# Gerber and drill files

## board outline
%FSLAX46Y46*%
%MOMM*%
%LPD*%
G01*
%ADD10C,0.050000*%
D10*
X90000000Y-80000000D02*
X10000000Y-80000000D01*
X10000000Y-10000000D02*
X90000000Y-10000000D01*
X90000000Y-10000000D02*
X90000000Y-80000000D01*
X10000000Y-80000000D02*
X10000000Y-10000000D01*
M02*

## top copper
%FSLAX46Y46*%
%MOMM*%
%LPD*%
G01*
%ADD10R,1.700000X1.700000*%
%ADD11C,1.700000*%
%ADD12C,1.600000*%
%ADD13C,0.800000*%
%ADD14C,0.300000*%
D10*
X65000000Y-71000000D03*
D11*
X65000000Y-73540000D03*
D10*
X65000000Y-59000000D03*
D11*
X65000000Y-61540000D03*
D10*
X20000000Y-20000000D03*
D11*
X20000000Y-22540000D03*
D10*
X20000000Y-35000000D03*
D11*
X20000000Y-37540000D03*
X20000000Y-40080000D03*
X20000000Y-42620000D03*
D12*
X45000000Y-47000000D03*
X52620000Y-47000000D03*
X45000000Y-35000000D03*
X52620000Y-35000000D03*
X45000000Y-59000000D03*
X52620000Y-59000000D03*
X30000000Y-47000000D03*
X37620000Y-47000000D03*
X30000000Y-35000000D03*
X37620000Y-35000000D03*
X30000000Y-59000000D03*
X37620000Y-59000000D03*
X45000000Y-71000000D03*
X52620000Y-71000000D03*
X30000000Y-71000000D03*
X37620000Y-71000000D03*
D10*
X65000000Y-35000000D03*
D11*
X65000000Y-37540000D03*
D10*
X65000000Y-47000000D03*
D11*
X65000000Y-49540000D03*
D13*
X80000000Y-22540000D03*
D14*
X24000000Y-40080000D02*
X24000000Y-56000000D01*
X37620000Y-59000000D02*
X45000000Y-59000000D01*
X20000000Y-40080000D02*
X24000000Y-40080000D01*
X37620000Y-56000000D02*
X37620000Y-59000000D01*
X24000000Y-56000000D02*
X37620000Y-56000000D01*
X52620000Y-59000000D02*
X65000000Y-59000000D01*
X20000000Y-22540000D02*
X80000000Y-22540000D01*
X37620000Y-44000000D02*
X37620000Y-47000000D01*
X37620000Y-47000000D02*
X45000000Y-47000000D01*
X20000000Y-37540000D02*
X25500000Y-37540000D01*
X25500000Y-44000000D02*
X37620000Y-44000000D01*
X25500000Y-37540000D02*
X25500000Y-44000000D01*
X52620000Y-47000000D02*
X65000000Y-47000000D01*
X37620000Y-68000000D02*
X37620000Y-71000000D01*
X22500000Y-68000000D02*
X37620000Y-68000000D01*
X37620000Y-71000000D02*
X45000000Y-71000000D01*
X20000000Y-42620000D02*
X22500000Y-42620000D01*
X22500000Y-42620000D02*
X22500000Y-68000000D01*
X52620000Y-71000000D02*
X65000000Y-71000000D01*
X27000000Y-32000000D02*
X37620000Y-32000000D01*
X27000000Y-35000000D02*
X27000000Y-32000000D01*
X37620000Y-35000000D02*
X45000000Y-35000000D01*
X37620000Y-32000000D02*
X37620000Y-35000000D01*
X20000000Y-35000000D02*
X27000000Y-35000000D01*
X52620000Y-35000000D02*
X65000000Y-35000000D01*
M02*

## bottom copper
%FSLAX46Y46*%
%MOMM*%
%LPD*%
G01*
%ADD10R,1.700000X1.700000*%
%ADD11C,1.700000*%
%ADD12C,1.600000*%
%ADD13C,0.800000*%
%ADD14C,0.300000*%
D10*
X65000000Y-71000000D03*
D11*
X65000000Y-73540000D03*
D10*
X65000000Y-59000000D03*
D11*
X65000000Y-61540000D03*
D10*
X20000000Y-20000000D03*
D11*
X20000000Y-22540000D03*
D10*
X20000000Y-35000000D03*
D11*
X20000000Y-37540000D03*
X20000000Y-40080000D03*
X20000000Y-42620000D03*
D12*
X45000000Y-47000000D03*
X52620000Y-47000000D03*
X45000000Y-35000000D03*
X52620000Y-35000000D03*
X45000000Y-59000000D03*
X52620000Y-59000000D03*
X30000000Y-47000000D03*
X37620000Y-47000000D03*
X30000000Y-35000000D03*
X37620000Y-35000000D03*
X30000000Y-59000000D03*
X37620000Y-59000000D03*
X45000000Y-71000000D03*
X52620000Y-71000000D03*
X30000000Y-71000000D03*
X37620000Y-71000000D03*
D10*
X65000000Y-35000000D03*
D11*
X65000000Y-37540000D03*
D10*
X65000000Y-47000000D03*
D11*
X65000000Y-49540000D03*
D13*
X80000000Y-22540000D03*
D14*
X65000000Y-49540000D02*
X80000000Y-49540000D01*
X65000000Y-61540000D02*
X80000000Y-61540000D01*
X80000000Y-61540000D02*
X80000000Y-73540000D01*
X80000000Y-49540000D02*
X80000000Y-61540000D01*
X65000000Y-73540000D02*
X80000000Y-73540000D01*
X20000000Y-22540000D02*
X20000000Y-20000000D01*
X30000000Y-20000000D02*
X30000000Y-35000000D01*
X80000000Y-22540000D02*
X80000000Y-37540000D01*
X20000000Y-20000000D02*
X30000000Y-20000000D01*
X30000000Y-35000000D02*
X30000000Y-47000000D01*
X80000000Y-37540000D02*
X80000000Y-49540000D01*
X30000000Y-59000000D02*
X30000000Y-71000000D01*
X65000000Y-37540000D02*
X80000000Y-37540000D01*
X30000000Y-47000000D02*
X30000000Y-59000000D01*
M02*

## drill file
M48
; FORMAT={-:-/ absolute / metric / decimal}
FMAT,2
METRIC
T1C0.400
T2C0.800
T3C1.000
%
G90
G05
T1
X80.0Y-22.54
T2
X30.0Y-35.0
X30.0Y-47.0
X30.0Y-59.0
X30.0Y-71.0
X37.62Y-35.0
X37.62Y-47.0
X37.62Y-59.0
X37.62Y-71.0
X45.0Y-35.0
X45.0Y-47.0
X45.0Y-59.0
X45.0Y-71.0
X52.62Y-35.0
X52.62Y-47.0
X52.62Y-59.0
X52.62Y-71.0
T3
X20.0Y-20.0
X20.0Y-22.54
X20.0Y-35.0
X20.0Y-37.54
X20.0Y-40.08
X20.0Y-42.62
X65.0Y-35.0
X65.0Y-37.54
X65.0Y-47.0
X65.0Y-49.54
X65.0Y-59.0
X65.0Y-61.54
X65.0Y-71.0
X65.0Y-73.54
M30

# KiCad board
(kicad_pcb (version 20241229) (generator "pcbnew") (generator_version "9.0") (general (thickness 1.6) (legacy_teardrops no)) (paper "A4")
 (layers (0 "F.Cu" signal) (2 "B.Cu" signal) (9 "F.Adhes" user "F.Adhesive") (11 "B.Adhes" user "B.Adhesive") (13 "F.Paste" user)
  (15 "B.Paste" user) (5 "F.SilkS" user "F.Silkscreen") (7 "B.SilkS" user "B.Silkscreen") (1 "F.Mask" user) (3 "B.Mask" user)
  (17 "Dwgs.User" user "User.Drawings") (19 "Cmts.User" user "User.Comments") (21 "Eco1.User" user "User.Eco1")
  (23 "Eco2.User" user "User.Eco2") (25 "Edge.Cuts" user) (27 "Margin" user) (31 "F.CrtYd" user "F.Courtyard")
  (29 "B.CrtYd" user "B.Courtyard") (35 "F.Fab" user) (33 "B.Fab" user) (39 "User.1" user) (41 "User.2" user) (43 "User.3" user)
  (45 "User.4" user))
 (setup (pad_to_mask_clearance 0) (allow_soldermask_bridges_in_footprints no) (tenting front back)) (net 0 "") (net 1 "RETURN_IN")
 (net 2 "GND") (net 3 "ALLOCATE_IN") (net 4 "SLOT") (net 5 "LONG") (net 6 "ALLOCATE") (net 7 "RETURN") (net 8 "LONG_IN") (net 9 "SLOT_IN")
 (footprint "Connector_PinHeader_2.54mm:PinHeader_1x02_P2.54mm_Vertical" (layer "F.Cu") (at 65 71)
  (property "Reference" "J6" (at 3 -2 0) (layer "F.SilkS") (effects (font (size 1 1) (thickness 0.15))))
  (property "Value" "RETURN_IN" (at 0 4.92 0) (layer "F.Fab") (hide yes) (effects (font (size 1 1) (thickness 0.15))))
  (pad "1" thru_hole rect (at 0 0) (size 1.7 1.7) (drill 1) (layers "*.Cu" "*.Mask") (remove_unused_layers no) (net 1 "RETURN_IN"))
  (pad "2" thru_hole circle (at 0 2.54) (size 1.7 1.7) (drill 1) (layers "*.Cu" "*.Mask") (remove_unused_layers no) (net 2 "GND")))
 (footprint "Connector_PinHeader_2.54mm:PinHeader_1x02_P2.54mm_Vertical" (layer "F.Cu") (at 65 59)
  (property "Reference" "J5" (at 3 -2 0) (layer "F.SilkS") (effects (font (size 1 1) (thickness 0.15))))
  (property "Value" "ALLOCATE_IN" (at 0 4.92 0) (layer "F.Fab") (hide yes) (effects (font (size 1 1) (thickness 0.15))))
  (pad "1" thru_hole rect (at 0 0) (size 1.7 1.7) (drill 1) (layers "*.Cu" "*.Mask") (remove_unused_layers no) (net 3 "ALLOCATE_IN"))
  (pad "2" thru_hole circle (at 0 2.54) (size 1.7 1.7) (drill 1) (layers "*.Cu" "*.Mask") (remove_unused_layers no) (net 2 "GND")))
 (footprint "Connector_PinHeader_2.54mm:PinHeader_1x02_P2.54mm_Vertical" (layer "F.Cu") (at 20 20)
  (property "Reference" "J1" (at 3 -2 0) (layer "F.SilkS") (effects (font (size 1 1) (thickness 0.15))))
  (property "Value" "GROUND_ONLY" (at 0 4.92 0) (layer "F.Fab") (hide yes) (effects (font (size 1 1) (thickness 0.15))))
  (pad "1" thru_hole rect (at 0 0) (size 1.7 1.7) (drill 1) (layers "*.Cu" "*.Mask") (remove_unused_layers no) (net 2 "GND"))
  (pad "2" thru_hole circle (at 0 2.54) (size 1.7 1.7) (drill 1) (layers "*.Cu" "*.Mask") (remove_unused_layers no) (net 2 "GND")))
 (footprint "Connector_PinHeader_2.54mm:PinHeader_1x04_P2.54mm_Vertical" (layer "F.Cu") (at 20 35)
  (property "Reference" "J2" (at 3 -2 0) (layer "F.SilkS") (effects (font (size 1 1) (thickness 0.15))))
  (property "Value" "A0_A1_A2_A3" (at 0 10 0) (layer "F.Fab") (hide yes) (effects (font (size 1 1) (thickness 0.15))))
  (pad "1" thru_hole rect (at 0 0) (size 1.7 1.7) (drill 1) (layers "*.Cu" "*.Mask") (remove_unused_layers no) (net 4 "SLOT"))
  (pad "2" thru_hole circle (at 0 2.54) (size 1.7 1.7) (drill 1) (layers "*.Cu" "*.Mask") (remove_unused_layers no) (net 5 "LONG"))
  (pad "3" thru_hole circle (at 0 5.08) (size 1.7 1.7) (drill 1) (layers "*.Cu" "*.Mask") (remove_unused_layers no) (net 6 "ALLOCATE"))
  (pad "4" thru_hole circle (at 0 7.62) (size 1.7 1.7) (drill 1) (layers "*.Cu" "*.Mask") (remove_unused_layers no) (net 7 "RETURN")))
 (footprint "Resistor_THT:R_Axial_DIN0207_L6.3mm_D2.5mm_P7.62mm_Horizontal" (layer "F.Cu") (at 45 47)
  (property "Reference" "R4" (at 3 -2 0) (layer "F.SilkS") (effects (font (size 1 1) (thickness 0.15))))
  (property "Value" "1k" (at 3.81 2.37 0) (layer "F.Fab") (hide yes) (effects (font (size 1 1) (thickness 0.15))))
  (pad "1" thru_hole circle (at 0 0) (size 1.6 1.6) (drill 0.8) (layers "*.Cu" "*.Mask") (remove_unused_layers no) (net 5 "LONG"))
  (pad "2" thru_hole circle (at 7.62 0) (size 1.6 1.6) (drill 0.8) (layers "*.Cu" "*.Mask") (remove_unused_layers no) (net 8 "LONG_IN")))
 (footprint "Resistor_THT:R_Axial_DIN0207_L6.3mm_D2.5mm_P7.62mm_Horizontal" (layer "F.Cu") (at 45 35)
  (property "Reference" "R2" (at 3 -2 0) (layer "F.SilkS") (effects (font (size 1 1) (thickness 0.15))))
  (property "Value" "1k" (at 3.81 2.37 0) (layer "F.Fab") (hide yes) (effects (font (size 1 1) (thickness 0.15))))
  (pad "1" thru_hole circle (at 0 0) (size 1.6 1.6) (drill 0.8) (layers "*.Cu" "*.Mask") (remove_unused_layers no) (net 4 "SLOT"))
  (pad "2" thru_hole circle (at 7.62 0) (size 1.6 1.6) (drill 0.8) (layers "*.Cu" "*.Mask") (remove_unused_layers no) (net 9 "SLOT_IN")))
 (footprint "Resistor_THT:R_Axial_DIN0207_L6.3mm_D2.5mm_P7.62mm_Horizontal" (layer "F.Cu") (at 45 59)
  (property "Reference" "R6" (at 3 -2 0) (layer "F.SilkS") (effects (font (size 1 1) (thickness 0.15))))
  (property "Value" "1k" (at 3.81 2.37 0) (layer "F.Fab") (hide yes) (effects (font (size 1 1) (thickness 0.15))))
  (pad "1" thru_hole circle (at 0 0) (size 1.6 1.6) (drill 0.8) (layers "*.Cu" "*.Mask") (remove_unused_layers no) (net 6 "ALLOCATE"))
  (pad "2" thru_hole circle (at 7.62 0) (size 1.6 1.6) (drill 0.8) (layers "*.Cu" "*.Mask") (remove_unused_layers no) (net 3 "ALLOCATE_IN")))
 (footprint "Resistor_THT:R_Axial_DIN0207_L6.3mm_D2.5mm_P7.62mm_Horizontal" (layer "F.Cu") (at 30 47)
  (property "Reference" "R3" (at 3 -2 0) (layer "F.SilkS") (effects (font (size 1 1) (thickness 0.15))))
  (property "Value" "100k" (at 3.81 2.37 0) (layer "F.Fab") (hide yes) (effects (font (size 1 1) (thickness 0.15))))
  (pad "1" thru_hole circle (at 0 0) (size 1.6 1.6) (drill 0.8) (layers "*.Cu" "*.Mask") (remove_unused_layers no) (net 2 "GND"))
  (pad "2" thru_hole circle (at 7.62 0) (size 1.6 1.6) (drill 0.8) (layers "*.Cu" "*.Mask") (remove_unused_layers no) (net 5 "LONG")))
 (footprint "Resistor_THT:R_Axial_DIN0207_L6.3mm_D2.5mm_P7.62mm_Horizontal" (layer "F.Cu") (at 30 35)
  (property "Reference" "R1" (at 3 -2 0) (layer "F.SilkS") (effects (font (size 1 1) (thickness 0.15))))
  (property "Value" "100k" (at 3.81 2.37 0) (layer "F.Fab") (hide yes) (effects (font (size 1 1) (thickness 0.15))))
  (pad "1" thru_hole circle (at 0 0) (size 1.6 1.6) (drill 0.8) (layers "*.Cu" "*.Mask") (remove_unused_layers no) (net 2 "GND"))
  (pad "2" thru_hole circle (at 7.62 0) (size 1.6 1.6) (drill 0.8) (layers "*.Cu" "*.Mask") (remove_unused_layers no) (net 4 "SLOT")))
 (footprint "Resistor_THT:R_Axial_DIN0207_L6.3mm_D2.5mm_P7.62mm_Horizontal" (layer "F.Cu") (at 30 59)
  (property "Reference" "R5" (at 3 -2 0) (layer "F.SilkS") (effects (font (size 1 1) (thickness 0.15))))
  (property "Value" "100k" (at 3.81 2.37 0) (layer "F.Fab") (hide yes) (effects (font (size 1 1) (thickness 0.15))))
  (pad "1" thru_hole circle (at 0 0) (size 1.6 1.6) (drill 0.8) (layers "*.Cu" "*.Mask") (remove_unused_layers no) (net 2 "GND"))
  (pad "2" thru_hole circle (at 7.62 0) (size 1.6 1.6) (drill 0.8) (layers "*.Cu" "*.Mask") (remove_unused_layers no) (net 6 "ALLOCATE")))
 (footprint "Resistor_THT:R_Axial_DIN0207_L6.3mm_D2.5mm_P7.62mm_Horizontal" (layer "F.Cu") (at 45 71)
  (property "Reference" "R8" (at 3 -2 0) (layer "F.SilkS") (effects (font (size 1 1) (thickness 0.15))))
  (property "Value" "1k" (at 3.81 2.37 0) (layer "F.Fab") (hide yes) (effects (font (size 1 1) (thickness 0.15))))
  (pad "1" thru_hole circle (at 0 0) (size 1.6 1.6) (drill 0.8) (layers "*.Cu" "*.Mask") (remove_unused_layers no) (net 7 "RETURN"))
  (pad "2" thru_hole circle (at 7.62 0) (size 1.6 1.6) (drill 0.8) (layers "*.Cu" "*.Mask") (remove_unused_layers no) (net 1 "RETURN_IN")))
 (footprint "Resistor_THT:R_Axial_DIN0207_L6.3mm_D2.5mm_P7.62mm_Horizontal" (layer "F.Cu") (at 30 71)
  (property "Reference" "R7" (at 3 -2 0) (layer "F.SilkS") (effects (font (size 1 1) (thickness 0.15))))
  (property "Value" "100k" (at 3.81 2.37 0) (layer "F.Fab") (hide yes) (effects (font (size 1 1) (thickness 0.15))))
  (pad "1" thru_hole circle (at 0 0) (size 1.6 1.6) (drill 0.8) (layers "*.Cu" "*.Mask") (remove_unused_layers no) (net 2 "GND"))
  (pad "2" thru_hole circle (at 7.62 0) (size 1.6 1.6) (drill 0.8) (layers "*.Cu" "*.Mask") (remove_unused_layers no) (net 7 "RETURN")))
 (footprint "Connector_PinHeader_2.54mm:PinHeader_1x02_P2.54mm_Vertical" (layer "F.Cu") (at 65 35)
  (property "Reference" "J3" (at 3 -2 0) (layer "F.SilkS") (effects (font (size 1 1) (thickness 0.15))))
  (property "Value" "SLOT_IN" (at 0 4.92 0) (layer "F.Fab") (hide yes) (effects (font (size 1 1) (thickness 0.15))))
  (pad "1" thru_hole rect (at 0 0) (size 1.7 1.7) (drill 1) (layers "*.Cu" "*.Mask") (remove_unused_layers no) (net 9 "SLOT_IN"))
  (pad "2" thru_hole circle (at 0 2.54) (size 1.7 1.7) (drill 1) (layers "*.Cu" "*.Mask") (remove_unused_layers no) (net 2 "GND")))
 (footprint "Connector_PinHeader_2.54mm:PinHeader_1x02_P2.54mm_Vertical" (layer "F.Cu") (at 65 47)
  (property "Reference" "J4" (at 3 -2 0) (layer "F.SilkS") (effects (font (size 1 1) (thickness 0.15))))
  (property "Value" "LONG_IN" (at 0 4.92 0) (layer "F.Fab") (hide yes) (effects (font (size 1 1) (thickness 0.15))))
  (pad "1" thru_hole rect (at 0 0) (size 1.7 1.7) (drill 1) (layers "*.Cu" "*.Mask") (remove_unused_layers no) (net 8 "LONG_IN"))
  (pad "2" thru_hole circle (at 0 2.54) (size 1.7 1.7) (drill 1) (layers "*.Cu" "*.Mask") (remove_unused_layers no) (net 2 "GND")))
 (gr_line (start 90 80) (end 10 80) (stroke (width 0.05) (type default)) (layer "Edge.Cuts"))
 (gr_line (start 10 10) (end 90 10) (stroke (width 0.05) (type default)) (layer "Edge.Cuts"))
 (gr_line (start 90 10) (end 90 80) (stroke (width 0.05) (type default)) (layer "Edge.Cuts"))
 (gr_line (start 10 80) (end 10 10) (stroke (width 0.05) (type default)) (layer "Edge.Cuts"))
 (segment (start 24 40.08) (end 24 56) (width 0.3) (layer "F.Cu") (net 6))
 (segment (start 37.62 59) (end 45 59) (width 0.3) (layer "F.Cu") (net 6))
 (segment (start 20 40.08) (end 24 40.08) (width 0.3) (layer "F.Cu") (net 6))
 (segment (start 37.62 56) (end 37.62 59) (width 0.3) (layer "F.Cu") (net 6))
 (segment (start 24 56) (end 37.62 56) (width 0.3) (layer "F.Cu") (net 6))
 (segment (start 52.62 59) (end 65 59) (width 0.3) (layer "F.Cu") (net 3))
 (segment (start 20 22.54) (end 80 22.54) (width 0.3) (layer "F.Cu") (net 2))
 (via (at 80 22.54) (size 0.8) (drill 0.4) (layers "F.Cu" "B.Cu") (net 2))
 (segment (start 65 49.54) (end 80 49.54) (width 0.3) (layer "B.Cu") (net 2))
 (segment (start 65 61.54) (end 80 61.54) (width 0.3) (layer "B.Cu") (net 2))
 (segment (start 80 61.54) (end 80 73.54) (width 0.3) (layer "B.Cu") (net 2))
 (segment (start 80 49.54) (end 80 61.54) (width 0.3) (layer "B.Cu") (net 2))
 (segment (start 65 73.54) (end 80 73.54) (width 0.3) (layer "B.Cu") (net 2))
 (segment (start 20 22.54) (end 20 20) (width 0.3) (layer "B.Cu") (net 2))
 (segment (start 30 20) (end 30 35) (width 0.3) (layer "B.Cu") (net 2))
 (segment (start 80 22.54) (end 80 37.54) (width 0.3) (layer "B.Cu") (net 2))
 (segment (start 20 20) (end 30 20) (width 0.3) (layer "B.Cu") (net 2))
 (segment (start 30 35) (end 30 47) (width 0.3) (layer "B.Cu") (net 2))
 (segment (start 80 37.54) (end 80 49.54) (width 0.3) (layer "B.Cu") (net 2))
 (segment (start 30 59) (end 30 71) (width 0.3) (layer "B.Cu") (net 2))
 (segment (start 65 37.54) (end 80 37.54) (width 0.3) (layer "B.Cu") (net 2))
 (segment (start 30 47) (end 30 59) (width 0.3) (layer "B.Cu") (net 2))
 (segment (start 37.62 44) (end 37.62 47) (width 0.3) (layer "F.Cu") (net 5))
 (segment (start 37.62 47) (end 45 47) (width 0.3) (layer "F.Cu") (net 5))
 (segment (start 20 37.54) (end 25.5 37.54) (width 0.3) (layer "F.Cu") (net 5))
 (segment (start 25.5 44) (end 37.62 44) (width 0.3) (layer "F.Cu") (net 5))
 (segment (start 25.5 37.54) (end 25.5 44) (width 0.3) (layer "F.Cu") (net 5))
 (segment (start 52.62 47) (end 65 47) (width 0.3) (layer "F.Cu") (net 8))
 (segment (start 37.62 68) (end 37.62 71) (width 0.3) (layer "F.Cu") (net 7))
 (segment (start 22.5 68) (end 37.62 68) (width 0.3) (layer "F.Cu") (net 7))
 (segment (start 37.62 71) (end 45 71) (width 0.3) (layer "F.Cu") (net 7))
 (segment (start 20 42.62) (end 22.5 42.62) (width 0.3) (layer "F.Cu") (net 7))
 (segment (start 22.5 42.62) (end 22.5 68) (width 0.3) (layer "F.Cu") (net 7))
 (segment (start 52.62 71) (end 65 71) (width 0.3) (layer "F.Cu") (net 1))
 (segment (start 27 32) (end 37.62 32) (width 0.3) (layer "F.Cu") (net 4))
 (segment (start 27 35) (end 27 32) (width 0.3) (layer "F.Cu") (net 4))
 (segment (start 37.62 35) (end 45 35) (width 0.3) (layer "F.Cu") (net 4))
 (segment (start 37.62 32) (end 37.62 35) (width 0.3) (layer "F.Cu") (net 4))
 (segment (start 20 35) (end 27 35) (width 0.3) (layer "F.Cu") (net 4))
 (segment (start 52.62 35) (end 65 35) (width 0.3) (layer "F.Cu") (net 9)))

